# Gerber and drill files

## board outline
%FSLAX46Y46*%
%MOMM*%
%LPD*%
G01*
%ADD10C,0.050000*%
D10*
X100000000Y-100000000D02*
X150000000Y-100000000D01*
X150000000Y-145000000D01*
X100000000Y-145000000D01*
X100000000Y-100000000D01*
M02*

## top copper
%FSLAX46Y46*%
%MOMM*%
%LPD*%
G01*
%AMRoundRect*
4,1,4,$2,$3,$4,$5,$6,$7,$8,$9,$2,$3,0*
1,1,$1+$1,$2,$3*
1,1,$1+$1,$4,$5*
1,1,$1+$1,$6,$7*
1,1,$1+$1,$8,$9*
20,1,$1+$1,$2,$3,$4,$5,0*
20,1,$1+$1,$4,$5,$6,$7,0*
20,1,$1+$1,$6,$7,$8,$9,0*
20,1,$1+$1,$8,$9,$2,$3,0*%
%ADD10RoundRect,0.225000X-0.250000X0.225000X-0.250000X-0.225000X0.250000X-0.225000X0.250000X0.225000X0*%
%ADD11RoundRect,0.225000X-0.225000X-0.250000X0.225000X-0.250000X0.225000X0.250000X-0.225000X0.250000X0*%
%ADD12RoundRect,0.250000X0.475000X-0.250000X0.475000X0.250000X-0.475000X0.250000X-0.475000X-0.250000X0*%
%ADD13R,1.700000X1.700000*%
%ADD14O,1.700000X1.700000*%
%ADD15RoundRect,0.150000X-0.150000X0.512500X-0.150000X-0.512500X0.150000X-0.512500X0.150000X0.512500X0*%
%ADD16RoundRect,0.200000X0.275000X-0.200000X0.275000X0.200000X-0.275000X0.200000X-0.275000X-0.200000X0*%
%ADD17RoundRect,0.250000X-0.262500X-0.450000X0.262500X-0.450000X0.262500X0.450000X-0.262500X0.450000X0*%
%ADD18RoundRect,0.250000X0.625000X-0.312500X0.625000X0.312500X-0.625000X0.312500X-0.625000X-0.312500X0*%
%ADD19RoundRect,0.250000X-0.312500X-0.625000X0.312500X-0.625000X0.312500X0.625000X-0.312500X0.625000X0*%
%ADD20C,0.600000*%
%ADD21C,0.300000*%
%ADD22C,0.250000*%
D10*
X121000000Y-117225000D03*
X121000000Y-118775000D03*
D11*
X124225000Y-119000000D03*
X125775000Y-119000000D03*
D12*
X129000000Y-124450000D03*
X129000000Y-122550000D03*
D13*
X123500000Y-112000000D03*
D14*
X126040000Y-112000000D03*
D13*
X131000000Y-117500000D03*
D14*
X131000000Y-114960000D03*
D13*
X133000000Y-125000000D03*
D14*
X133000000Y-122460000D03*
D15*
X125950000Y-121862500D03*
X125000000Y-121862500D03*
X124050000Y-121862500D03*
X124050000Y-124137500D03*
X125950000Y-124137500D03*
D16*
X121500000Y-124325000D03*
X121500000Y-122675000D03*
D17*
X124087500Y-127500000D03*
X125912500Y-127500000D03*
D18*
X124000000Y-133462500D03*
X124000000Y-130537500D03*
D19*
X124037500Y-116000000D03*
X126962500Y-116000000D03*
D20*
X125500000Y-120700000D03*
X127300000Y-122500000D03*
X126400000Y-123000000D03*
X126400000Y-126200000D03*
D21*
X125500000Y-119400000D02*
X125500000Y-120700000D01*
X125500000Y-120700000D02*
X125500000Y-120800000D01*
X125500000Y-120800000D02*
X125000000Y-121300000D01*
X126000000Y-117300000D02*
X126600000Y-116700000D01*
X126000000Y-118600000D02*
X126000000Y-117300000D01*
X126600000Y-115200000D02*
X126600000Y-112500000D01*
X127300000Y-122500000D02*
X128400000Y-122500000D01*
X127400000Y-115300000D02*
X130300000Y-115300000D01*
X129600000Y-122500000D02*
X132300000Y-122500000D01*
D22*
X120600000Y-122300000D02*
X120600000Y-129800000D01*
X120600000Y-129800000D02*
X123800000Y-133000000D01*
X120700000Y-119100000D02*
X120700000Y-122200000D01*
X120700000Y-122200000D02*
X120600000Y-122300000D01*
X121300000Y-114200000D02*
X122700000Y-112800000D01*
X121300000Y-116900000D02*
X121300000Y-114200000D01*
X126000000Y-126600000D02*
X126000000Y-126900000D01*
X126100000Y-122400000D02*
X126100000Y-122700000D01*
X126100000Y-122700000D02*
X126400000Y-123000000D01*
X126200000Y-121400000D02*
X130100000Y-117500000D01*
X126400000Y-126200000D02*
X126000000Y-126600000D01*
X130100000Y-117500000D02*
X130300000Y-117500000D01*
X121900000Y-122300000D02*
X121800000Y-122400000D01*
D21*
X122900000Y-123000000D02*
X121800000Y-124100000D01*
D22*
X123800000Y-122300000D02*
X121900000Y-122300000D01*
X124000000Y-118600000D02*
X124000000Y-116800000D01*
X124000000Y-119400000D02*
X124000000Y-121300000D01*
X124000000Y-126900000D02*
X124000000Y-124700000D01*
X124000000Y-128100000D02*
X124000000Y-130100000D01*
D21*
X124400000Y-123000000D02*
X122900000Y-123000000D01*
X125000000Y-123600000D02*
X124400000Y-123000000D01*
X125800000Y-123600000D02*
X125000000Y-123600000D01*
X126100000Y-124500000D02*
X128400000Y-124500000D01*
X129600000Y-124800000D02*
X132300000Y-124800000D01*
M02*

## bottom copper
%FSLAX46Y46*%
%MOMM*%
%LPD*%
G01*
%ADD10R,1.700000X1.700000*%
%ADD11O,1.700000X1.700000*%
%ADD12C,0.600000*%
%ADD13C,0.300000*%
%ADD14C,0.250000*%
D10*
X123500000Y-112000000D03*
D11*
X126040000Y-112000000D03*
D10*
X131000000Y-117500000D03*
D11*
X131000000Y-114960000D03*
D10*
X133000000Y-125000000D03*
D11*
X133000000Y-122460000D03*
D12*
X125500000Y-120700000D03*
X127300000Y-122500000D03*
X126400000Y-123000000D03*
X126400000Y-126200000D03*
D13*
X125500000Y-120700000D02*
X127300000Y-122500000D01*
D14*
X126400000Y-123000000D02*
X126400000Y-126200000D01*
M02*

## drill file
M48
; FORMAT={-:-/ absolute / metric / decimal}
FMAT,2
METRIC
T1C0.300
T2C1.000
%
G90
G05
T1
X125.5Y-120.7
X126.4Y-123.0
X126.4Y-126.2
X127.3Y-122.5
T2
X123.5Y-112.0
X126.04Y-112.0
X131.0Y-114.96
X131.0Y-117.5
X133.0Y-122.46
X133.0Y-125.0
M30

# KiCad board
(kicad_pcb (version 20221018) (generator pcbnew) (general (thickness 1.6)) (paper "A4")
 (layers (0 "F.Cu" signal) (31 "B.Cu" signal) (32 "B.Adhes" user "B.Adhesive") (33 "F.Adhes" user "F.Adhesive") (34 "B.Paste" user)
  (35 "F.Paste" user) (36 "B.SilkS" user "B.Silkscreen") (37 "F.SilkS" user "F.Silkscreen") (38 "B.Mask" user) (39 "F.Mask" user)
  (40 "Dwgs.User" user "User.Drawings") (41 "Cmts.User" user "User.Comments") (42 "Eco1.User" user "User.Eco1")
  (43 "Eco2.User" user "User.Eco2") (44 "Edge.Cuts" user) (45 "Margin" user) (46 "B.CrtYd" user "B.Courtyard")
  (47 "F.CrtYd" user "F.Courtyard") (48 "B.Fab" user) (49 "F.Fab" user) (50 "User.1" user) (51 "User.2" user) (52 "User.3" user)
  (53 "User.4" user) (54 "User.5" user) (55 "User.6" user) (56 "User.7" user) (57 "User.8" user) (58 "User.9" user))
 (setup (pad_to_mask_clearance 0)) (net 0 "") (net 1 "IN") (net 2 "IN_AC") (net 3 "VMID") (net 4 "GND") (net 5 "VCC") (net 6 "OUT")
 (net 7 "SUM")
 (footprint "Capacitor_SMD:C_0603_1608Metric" (layer "F.Cu") (at 121 118 -90)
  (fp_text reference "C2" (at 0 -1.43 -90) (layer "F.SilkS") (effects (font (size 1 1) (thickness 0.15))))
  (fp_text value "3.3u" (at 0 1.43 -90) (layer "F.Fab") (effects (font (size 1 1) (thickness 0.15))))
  (pad "1" smd roundrect (at -0.775 0 270) (size 0.9 0.95) (layers "F.Cu" "F.Paste" "F.Mask") (roundrect_rratio 0.25) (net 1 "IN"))
  (pad "2" smd roundrect (at 0.775 0 270) (size 0.9 0.95) (layers "F.Cu" "F.Paste" "F.Mask") (roundrect_rratio 0.25) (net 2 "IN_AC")))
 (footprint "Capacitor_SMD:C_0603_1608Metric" (layer "F.Cu") (at 125 119)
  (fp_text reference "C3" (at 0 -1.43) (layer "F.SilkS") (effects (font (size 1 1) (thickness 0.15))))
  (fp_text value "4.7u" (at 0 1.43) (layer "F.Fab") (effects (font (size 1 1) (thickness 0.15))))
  (pad "1" smd roundrect (at -0.775 0) (size 0.9 0.95) (layers "F.Cu" "F.Paste" "F.Mask") (roundrect_rratio 0.25) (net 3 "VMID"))
  (pad "2" smd roundrect (at 0.775 0) (size 0.9 0.95) (layers "F.Cu" "F.Paste" "F.Mask") (roundrect_rratio 0.25) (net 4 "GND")))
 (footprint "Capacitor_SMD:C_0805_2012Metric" (layer "F.Cu") (at 129 123.5 90)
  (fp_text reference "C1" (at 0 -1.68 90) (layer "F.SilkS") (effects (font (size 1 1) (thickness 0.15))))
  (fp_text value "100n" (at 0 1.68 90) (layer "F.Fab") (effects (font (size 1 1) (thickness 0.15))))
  (pad "1" smd roundrect (at -0.95 0 90) (size 1 1.45) (layers "F.Cu" "F.Paste" "F.Mask") (roundrect_rratio 0.25) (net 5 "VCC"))
  (pad "2" smd roundrect (at 0.95 0 90) (size 1 1.45) (layers "F.Cu" "F.Paste" "F.Mask") (roundrect_rratio 0.25) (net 4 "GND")))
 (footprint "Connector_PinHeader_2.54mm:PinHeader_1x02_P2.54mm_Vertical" (layer "F.Cu") (at 123.5 112 90)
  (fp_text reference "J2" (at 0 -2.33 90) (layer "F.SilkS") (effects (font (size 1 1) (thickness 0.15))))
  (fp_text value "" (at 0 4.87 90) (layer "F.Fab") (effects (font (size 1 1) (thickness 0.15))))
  (pad "1" thru_hole rect (at 0 0 90) (size 1.7 1.7) (drill 1) (layers "*.Cu" "*.Mask") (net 1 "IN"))
  (pad "2" thru_hole oval (at 0 2.54 90) (size 1.7 1.7) (drill 1) (layers "*.Cu" "*.Mask") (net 4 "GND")))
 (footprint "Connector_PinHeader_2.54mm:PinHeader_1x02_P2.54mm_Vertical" (layer "F.Cu") (at 131 117.5 180)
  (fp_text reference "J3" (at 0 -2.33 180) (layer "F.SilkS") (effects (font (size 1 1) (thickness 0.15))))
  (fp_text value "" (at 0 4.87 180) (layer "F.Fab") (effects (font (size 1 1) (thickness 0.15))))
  (pad "1" thru_hole rect (at 0 0 180) (size 1.7 1.7) (drill 1) (layers "*.Cu" "*.Mask") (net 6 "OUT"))
  (pad "2" thru_hole oval (at 0 2.54 180) (size 1.7 1.7) (drill 1) (layers "*.Cu" "*.Mask") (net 4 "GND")))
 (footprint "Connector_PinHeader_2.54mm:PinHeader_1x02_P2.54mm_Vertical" (layer "F.Cu") (at 133 125 180)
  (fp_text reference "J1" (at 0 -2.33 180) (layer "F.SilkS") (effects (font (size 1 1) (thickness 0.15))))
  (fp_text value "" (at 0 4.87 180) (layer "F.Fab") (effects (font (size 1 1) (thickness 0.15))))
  (pad "1" thru_hole rect (at 0 0 180) (size 1.7 1.7) (drill 1) (layers "*.Cu" "*.Mask") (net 5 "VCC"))
  (pad "2" thru_hole oval (at 0 2.54 180) (size 1.7 1.7) (drill 1) (layers "*.Cu" "*.Mask") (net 4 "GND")))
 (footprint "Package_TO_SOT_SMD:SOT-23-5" (layer "F.Cu") (at 125 123 -90)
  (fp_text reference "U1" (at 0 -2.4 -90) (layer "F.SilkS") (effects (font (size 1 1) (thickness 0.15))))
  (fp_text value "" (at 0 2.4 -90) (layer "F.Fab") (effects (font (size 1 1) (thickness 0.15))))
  (pad "1" smd roundrect (at -1.1375 -0.95 270) (size 1.325 0.6) (layers "F.Cu" "F.Paste" "F.Mask") (roundrect_rratio 0.25) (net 6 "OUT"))
  (pad "2" smd roundrect (at -1.1375 0 270) (size 1.325 0.6) (layers "F.Cu" "F.Paste" "F.Mask") (roundrect_rratio 0.25) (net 4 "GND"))
  (pad "3" smd roundrect (at -1.1375 0.95 270) (size 1.325 0.6) (layers "F.Cu" "F.Paste" "F.Mask") (roundrect_rratio 0.25) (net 3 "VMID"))
  (pad "4" smd roundrect (at 1.1375 0.95 270) (size 1.325 0.6) (layers "F.Cu" "F.Paste" "F.Mask") (roundrect_rratio 0.25) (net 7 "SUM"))
  (pad "5" smd roundrect (at 1.1375 -0.95 270) (size 1.325 0.6) (layers "F.Cu" "F.Paste" "F.Mask") (roundrect_rratio 0.25) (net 5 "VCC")))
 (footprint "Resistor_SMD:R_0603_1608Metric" (layer "F.Cu") (at 121.5 123.5 90)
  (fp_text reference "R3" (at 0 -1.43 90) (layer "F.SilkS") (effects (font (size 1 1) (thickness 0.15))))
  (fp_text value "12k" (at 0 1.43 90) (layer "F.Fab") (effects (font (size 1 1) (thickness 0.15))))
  (pad "1" smd roundrect (at -0.825 0 90) (size 0.8 0.95) (layers "F.Cu" "F.Paste" "F.Mask") (roundrect_rratio 0.25) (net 5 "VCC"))
  (pad "2" smd roundrect (at 0.825 0 90) (size 0.8 0.95) (layers "F.Cu" "F.Paste" "F.Mask") (roundrect_rratio 0.25) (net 3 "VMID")))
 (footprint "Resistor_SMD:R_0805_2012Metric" (layer "F.Cu") (at 125 127.5)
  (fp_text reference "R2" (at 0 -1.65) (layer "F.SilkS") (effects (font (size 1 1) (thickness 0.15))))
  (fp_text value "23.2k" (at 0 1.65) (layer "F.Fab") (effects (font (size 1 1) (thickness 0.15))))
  (pad "1" smd roundrect (at -0.9125 0) (size 1.025 1.4) (layers "F.Cu" "F.Paste" "F.Mask") (roundrect_rratio 0.243902) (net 7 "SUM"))
  (pad "2" smd roundrect (at 0.9125 0) (size 1.025 1.4) (layers "F.Cu" "F.Paste" "F.Mask") (roundrect_rratio 0.243902) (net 6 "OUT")))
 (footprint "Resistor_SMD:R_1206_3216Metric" (layer "F.Cu") (at 124 132 90)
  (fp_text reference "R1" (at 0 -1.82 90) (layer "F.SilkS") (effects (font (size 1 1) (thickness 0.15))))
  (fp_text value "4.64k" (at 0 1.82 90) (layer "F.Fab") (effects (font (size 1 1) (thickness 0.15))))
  (pad "1" smd roundrect (at -1.4625 0 90) (size 1.125 1.75) (layers "F.Cu" "F.Paste" "F.Mask") (roundrect_rratio 0.222222) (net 2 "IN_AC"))
  (pad "2" smd roundrect (at 1.4625 0 90) (size 1.125 1.75) (layers "F.Cu" "F.Paste" "F.Mask") (roundrect_rratio 0.222222) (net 7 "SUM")))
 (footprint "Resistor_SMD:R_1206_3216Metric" (layer "F.Cu") (at 125.5 116)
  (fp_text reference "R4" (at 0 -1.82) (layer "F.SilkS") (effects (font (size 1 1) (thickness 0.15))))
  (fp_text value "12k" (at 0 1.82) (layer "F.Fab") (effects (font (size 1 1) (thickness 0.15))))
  (pad "1" smd roundrect (at -1.4625 0) (size 1.125 1.75) (layers "F.Cu" "F.Paste" "F.Mask") (roundrect_rratio 0.222222) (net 3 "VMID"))
  (pad "2" smd roundrect (at 1.4625 0) (size 1.125 1.75) (layers "F.Cu" "F.Paste" "F.Mask") (roundrect_rratio 0.222222) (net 4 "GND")))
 (gr_rect (start 100 100) (end 150 145) (stroke (width 0.05) (type default)) (fill none) (layer "Edge.Cuts"))
 (segment (start 125.5 119.4) (end 125.5 120.7) (width 0.3) (layer "F.Cu") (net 4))
 (segment (start 125.5 120.7) (end 125.5 120.8) (width 0.3) (layer "F.Cu") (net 4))
 (segment (start 125.5 120.8) (end 125 121.3) (width 0.3) (layer "F.Cu") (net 4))
 (segment (start 126 117.3) (end 126.6 116.7) (width 0.3) (layer "F.Cu") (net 4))
 (segment (start 126 118.6) (end 126 117.3) (width 0.3) (layer "F.Cu") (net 4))
 (segment (start 126.6 115.2) (end 126.6 112.5) (width 0.3) (layer "F.Cu") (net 4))
 (segment (start 127.3 122.5) (end 128.4 122.5) (width 0.3) (layer "F.Cu") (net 4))
 (segment (start 127.4 115.3) (end 130.3 115.3) (width 0.3) (layer "F.Cu") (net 4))
 (segment (start 129.6 122.5) (end 132.3 122.5) (width 0.3) (layer "F.Cu") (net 4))
 (via (at 125.5 120.7) (size 0.6) (drill 0.3) (layers "F.Cu" "B.Cu") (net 4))
 (via (at 127.3 122.5) (size 0.6) (drill 0.3) (layers "F.Cu" "B.Cu") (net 4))
 (segment (start 120.6 122.3) (end 120.6 129.8) (width 0.25) (layer "F.Cu") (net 2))
 (segment (start 120.6 129.8) (end 123.8 133) (width 0.25) (layer "F.Cu") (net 2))
 (segment (start 120.7 119.1) (end 120.7 122.2) (width 0.25) (layer "F.Cu") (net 2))
 (segment (start 120.7 122.2) (end 120.6 122.3) (width 0.25) (layer "F.Cu") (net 2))
 (segment (start 121.3 114.2) (end 122.7 112.8) (width 0.25) (layer "F.Cu") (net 1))
 (segment (start 121.3 116.9) (end 121.3 114.2) (width 0.25) (layer "F.Cu") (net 1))
 (segment (start 125.5 120.7) (end 127.3 122.5) (width 0.3) (layer "B.Cu") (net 4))
 (segment (start 126 126.6) (end 126 126.9) (width 0.25) (layer "F.Cu") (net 6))
 (segment (start 126.1 122.4) (end 126.1 122.7) (width 0.25) (layer "F.Cu") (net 6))
 (segment (start 126.1 122.7) (end 126.4 123) (width 0.25) (layer "F.Cu") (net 6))
 (segment (start 126.2 121.4) (end 130.1 117.5) (width 0.25) (layer "F.Cu") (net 6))
 (segment (start 126.4 126.2) (end 126 126.6) (width 0.25) (layer "F.Cu") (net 6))
 (segment (start 130.1 117.5) (end 130.3 117.5) (width 0.25) (layer "F.Cu") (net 6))
 (via (at 126.4 123) (size 0.6) (drill 0.3) (layers "F.Cu" "B.Cu") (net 6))
 (via (at 126.4 126.2) (size 0.6) (drill 0.3) (layers "F.Cu" "B.Cu") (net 6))
 (segment (start 121.9 122.3) (end 121.8 122.4) (width 0.25) (layer "F.Cu") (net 3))
 (segment (start 122.9 123) (end 121.8 124.1) (width 0.3) (layer "F.Cu") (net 5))
 (segment (start 123.8 122.3) (end 121.9 122.3) (width 0.25) (layer "F.Cu") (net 3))
 (segment (start 124 118.6) (end 124 116.8) (width 0.25) (layer "F.Cu") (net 3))
 (segment (start 124 119.4) (end 124 121.3) (width 0.25) (layer "F.Cu") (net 3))
 (segment (start 124 126.9) (end 124 124.7) (width 0.25) (layer "F.Cu") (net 7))
 (segment (start 124 128.1) (end 124 130.1) (width 0.25) (layer "F.Cu") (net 7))
 (segment (start 124.4 123) (end 122.9 123) (width 0.3) (layer "F.Cu") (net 5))
 (segment (start 125 123.6) (end 124.4 123) (width 0.3) (layer "F.Cu") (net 5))
 (segment (start 125.8 123.6) (end 125 123.6) (width 0.3) (layer "F.Cu") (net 5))
 (segment (start 126.1 124.5) (end 128.4 124.5) (width 0.3) (layer "F.Cu") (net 5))
 (segment (start 126.4 123) (end 126.4 126.2) (width 0.25) (layer "B.Cu") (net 6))
 (segment (start 129.6 124.8) (end 132.3 124.8) (width 0.3) (layer "F.Cu") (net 5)))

